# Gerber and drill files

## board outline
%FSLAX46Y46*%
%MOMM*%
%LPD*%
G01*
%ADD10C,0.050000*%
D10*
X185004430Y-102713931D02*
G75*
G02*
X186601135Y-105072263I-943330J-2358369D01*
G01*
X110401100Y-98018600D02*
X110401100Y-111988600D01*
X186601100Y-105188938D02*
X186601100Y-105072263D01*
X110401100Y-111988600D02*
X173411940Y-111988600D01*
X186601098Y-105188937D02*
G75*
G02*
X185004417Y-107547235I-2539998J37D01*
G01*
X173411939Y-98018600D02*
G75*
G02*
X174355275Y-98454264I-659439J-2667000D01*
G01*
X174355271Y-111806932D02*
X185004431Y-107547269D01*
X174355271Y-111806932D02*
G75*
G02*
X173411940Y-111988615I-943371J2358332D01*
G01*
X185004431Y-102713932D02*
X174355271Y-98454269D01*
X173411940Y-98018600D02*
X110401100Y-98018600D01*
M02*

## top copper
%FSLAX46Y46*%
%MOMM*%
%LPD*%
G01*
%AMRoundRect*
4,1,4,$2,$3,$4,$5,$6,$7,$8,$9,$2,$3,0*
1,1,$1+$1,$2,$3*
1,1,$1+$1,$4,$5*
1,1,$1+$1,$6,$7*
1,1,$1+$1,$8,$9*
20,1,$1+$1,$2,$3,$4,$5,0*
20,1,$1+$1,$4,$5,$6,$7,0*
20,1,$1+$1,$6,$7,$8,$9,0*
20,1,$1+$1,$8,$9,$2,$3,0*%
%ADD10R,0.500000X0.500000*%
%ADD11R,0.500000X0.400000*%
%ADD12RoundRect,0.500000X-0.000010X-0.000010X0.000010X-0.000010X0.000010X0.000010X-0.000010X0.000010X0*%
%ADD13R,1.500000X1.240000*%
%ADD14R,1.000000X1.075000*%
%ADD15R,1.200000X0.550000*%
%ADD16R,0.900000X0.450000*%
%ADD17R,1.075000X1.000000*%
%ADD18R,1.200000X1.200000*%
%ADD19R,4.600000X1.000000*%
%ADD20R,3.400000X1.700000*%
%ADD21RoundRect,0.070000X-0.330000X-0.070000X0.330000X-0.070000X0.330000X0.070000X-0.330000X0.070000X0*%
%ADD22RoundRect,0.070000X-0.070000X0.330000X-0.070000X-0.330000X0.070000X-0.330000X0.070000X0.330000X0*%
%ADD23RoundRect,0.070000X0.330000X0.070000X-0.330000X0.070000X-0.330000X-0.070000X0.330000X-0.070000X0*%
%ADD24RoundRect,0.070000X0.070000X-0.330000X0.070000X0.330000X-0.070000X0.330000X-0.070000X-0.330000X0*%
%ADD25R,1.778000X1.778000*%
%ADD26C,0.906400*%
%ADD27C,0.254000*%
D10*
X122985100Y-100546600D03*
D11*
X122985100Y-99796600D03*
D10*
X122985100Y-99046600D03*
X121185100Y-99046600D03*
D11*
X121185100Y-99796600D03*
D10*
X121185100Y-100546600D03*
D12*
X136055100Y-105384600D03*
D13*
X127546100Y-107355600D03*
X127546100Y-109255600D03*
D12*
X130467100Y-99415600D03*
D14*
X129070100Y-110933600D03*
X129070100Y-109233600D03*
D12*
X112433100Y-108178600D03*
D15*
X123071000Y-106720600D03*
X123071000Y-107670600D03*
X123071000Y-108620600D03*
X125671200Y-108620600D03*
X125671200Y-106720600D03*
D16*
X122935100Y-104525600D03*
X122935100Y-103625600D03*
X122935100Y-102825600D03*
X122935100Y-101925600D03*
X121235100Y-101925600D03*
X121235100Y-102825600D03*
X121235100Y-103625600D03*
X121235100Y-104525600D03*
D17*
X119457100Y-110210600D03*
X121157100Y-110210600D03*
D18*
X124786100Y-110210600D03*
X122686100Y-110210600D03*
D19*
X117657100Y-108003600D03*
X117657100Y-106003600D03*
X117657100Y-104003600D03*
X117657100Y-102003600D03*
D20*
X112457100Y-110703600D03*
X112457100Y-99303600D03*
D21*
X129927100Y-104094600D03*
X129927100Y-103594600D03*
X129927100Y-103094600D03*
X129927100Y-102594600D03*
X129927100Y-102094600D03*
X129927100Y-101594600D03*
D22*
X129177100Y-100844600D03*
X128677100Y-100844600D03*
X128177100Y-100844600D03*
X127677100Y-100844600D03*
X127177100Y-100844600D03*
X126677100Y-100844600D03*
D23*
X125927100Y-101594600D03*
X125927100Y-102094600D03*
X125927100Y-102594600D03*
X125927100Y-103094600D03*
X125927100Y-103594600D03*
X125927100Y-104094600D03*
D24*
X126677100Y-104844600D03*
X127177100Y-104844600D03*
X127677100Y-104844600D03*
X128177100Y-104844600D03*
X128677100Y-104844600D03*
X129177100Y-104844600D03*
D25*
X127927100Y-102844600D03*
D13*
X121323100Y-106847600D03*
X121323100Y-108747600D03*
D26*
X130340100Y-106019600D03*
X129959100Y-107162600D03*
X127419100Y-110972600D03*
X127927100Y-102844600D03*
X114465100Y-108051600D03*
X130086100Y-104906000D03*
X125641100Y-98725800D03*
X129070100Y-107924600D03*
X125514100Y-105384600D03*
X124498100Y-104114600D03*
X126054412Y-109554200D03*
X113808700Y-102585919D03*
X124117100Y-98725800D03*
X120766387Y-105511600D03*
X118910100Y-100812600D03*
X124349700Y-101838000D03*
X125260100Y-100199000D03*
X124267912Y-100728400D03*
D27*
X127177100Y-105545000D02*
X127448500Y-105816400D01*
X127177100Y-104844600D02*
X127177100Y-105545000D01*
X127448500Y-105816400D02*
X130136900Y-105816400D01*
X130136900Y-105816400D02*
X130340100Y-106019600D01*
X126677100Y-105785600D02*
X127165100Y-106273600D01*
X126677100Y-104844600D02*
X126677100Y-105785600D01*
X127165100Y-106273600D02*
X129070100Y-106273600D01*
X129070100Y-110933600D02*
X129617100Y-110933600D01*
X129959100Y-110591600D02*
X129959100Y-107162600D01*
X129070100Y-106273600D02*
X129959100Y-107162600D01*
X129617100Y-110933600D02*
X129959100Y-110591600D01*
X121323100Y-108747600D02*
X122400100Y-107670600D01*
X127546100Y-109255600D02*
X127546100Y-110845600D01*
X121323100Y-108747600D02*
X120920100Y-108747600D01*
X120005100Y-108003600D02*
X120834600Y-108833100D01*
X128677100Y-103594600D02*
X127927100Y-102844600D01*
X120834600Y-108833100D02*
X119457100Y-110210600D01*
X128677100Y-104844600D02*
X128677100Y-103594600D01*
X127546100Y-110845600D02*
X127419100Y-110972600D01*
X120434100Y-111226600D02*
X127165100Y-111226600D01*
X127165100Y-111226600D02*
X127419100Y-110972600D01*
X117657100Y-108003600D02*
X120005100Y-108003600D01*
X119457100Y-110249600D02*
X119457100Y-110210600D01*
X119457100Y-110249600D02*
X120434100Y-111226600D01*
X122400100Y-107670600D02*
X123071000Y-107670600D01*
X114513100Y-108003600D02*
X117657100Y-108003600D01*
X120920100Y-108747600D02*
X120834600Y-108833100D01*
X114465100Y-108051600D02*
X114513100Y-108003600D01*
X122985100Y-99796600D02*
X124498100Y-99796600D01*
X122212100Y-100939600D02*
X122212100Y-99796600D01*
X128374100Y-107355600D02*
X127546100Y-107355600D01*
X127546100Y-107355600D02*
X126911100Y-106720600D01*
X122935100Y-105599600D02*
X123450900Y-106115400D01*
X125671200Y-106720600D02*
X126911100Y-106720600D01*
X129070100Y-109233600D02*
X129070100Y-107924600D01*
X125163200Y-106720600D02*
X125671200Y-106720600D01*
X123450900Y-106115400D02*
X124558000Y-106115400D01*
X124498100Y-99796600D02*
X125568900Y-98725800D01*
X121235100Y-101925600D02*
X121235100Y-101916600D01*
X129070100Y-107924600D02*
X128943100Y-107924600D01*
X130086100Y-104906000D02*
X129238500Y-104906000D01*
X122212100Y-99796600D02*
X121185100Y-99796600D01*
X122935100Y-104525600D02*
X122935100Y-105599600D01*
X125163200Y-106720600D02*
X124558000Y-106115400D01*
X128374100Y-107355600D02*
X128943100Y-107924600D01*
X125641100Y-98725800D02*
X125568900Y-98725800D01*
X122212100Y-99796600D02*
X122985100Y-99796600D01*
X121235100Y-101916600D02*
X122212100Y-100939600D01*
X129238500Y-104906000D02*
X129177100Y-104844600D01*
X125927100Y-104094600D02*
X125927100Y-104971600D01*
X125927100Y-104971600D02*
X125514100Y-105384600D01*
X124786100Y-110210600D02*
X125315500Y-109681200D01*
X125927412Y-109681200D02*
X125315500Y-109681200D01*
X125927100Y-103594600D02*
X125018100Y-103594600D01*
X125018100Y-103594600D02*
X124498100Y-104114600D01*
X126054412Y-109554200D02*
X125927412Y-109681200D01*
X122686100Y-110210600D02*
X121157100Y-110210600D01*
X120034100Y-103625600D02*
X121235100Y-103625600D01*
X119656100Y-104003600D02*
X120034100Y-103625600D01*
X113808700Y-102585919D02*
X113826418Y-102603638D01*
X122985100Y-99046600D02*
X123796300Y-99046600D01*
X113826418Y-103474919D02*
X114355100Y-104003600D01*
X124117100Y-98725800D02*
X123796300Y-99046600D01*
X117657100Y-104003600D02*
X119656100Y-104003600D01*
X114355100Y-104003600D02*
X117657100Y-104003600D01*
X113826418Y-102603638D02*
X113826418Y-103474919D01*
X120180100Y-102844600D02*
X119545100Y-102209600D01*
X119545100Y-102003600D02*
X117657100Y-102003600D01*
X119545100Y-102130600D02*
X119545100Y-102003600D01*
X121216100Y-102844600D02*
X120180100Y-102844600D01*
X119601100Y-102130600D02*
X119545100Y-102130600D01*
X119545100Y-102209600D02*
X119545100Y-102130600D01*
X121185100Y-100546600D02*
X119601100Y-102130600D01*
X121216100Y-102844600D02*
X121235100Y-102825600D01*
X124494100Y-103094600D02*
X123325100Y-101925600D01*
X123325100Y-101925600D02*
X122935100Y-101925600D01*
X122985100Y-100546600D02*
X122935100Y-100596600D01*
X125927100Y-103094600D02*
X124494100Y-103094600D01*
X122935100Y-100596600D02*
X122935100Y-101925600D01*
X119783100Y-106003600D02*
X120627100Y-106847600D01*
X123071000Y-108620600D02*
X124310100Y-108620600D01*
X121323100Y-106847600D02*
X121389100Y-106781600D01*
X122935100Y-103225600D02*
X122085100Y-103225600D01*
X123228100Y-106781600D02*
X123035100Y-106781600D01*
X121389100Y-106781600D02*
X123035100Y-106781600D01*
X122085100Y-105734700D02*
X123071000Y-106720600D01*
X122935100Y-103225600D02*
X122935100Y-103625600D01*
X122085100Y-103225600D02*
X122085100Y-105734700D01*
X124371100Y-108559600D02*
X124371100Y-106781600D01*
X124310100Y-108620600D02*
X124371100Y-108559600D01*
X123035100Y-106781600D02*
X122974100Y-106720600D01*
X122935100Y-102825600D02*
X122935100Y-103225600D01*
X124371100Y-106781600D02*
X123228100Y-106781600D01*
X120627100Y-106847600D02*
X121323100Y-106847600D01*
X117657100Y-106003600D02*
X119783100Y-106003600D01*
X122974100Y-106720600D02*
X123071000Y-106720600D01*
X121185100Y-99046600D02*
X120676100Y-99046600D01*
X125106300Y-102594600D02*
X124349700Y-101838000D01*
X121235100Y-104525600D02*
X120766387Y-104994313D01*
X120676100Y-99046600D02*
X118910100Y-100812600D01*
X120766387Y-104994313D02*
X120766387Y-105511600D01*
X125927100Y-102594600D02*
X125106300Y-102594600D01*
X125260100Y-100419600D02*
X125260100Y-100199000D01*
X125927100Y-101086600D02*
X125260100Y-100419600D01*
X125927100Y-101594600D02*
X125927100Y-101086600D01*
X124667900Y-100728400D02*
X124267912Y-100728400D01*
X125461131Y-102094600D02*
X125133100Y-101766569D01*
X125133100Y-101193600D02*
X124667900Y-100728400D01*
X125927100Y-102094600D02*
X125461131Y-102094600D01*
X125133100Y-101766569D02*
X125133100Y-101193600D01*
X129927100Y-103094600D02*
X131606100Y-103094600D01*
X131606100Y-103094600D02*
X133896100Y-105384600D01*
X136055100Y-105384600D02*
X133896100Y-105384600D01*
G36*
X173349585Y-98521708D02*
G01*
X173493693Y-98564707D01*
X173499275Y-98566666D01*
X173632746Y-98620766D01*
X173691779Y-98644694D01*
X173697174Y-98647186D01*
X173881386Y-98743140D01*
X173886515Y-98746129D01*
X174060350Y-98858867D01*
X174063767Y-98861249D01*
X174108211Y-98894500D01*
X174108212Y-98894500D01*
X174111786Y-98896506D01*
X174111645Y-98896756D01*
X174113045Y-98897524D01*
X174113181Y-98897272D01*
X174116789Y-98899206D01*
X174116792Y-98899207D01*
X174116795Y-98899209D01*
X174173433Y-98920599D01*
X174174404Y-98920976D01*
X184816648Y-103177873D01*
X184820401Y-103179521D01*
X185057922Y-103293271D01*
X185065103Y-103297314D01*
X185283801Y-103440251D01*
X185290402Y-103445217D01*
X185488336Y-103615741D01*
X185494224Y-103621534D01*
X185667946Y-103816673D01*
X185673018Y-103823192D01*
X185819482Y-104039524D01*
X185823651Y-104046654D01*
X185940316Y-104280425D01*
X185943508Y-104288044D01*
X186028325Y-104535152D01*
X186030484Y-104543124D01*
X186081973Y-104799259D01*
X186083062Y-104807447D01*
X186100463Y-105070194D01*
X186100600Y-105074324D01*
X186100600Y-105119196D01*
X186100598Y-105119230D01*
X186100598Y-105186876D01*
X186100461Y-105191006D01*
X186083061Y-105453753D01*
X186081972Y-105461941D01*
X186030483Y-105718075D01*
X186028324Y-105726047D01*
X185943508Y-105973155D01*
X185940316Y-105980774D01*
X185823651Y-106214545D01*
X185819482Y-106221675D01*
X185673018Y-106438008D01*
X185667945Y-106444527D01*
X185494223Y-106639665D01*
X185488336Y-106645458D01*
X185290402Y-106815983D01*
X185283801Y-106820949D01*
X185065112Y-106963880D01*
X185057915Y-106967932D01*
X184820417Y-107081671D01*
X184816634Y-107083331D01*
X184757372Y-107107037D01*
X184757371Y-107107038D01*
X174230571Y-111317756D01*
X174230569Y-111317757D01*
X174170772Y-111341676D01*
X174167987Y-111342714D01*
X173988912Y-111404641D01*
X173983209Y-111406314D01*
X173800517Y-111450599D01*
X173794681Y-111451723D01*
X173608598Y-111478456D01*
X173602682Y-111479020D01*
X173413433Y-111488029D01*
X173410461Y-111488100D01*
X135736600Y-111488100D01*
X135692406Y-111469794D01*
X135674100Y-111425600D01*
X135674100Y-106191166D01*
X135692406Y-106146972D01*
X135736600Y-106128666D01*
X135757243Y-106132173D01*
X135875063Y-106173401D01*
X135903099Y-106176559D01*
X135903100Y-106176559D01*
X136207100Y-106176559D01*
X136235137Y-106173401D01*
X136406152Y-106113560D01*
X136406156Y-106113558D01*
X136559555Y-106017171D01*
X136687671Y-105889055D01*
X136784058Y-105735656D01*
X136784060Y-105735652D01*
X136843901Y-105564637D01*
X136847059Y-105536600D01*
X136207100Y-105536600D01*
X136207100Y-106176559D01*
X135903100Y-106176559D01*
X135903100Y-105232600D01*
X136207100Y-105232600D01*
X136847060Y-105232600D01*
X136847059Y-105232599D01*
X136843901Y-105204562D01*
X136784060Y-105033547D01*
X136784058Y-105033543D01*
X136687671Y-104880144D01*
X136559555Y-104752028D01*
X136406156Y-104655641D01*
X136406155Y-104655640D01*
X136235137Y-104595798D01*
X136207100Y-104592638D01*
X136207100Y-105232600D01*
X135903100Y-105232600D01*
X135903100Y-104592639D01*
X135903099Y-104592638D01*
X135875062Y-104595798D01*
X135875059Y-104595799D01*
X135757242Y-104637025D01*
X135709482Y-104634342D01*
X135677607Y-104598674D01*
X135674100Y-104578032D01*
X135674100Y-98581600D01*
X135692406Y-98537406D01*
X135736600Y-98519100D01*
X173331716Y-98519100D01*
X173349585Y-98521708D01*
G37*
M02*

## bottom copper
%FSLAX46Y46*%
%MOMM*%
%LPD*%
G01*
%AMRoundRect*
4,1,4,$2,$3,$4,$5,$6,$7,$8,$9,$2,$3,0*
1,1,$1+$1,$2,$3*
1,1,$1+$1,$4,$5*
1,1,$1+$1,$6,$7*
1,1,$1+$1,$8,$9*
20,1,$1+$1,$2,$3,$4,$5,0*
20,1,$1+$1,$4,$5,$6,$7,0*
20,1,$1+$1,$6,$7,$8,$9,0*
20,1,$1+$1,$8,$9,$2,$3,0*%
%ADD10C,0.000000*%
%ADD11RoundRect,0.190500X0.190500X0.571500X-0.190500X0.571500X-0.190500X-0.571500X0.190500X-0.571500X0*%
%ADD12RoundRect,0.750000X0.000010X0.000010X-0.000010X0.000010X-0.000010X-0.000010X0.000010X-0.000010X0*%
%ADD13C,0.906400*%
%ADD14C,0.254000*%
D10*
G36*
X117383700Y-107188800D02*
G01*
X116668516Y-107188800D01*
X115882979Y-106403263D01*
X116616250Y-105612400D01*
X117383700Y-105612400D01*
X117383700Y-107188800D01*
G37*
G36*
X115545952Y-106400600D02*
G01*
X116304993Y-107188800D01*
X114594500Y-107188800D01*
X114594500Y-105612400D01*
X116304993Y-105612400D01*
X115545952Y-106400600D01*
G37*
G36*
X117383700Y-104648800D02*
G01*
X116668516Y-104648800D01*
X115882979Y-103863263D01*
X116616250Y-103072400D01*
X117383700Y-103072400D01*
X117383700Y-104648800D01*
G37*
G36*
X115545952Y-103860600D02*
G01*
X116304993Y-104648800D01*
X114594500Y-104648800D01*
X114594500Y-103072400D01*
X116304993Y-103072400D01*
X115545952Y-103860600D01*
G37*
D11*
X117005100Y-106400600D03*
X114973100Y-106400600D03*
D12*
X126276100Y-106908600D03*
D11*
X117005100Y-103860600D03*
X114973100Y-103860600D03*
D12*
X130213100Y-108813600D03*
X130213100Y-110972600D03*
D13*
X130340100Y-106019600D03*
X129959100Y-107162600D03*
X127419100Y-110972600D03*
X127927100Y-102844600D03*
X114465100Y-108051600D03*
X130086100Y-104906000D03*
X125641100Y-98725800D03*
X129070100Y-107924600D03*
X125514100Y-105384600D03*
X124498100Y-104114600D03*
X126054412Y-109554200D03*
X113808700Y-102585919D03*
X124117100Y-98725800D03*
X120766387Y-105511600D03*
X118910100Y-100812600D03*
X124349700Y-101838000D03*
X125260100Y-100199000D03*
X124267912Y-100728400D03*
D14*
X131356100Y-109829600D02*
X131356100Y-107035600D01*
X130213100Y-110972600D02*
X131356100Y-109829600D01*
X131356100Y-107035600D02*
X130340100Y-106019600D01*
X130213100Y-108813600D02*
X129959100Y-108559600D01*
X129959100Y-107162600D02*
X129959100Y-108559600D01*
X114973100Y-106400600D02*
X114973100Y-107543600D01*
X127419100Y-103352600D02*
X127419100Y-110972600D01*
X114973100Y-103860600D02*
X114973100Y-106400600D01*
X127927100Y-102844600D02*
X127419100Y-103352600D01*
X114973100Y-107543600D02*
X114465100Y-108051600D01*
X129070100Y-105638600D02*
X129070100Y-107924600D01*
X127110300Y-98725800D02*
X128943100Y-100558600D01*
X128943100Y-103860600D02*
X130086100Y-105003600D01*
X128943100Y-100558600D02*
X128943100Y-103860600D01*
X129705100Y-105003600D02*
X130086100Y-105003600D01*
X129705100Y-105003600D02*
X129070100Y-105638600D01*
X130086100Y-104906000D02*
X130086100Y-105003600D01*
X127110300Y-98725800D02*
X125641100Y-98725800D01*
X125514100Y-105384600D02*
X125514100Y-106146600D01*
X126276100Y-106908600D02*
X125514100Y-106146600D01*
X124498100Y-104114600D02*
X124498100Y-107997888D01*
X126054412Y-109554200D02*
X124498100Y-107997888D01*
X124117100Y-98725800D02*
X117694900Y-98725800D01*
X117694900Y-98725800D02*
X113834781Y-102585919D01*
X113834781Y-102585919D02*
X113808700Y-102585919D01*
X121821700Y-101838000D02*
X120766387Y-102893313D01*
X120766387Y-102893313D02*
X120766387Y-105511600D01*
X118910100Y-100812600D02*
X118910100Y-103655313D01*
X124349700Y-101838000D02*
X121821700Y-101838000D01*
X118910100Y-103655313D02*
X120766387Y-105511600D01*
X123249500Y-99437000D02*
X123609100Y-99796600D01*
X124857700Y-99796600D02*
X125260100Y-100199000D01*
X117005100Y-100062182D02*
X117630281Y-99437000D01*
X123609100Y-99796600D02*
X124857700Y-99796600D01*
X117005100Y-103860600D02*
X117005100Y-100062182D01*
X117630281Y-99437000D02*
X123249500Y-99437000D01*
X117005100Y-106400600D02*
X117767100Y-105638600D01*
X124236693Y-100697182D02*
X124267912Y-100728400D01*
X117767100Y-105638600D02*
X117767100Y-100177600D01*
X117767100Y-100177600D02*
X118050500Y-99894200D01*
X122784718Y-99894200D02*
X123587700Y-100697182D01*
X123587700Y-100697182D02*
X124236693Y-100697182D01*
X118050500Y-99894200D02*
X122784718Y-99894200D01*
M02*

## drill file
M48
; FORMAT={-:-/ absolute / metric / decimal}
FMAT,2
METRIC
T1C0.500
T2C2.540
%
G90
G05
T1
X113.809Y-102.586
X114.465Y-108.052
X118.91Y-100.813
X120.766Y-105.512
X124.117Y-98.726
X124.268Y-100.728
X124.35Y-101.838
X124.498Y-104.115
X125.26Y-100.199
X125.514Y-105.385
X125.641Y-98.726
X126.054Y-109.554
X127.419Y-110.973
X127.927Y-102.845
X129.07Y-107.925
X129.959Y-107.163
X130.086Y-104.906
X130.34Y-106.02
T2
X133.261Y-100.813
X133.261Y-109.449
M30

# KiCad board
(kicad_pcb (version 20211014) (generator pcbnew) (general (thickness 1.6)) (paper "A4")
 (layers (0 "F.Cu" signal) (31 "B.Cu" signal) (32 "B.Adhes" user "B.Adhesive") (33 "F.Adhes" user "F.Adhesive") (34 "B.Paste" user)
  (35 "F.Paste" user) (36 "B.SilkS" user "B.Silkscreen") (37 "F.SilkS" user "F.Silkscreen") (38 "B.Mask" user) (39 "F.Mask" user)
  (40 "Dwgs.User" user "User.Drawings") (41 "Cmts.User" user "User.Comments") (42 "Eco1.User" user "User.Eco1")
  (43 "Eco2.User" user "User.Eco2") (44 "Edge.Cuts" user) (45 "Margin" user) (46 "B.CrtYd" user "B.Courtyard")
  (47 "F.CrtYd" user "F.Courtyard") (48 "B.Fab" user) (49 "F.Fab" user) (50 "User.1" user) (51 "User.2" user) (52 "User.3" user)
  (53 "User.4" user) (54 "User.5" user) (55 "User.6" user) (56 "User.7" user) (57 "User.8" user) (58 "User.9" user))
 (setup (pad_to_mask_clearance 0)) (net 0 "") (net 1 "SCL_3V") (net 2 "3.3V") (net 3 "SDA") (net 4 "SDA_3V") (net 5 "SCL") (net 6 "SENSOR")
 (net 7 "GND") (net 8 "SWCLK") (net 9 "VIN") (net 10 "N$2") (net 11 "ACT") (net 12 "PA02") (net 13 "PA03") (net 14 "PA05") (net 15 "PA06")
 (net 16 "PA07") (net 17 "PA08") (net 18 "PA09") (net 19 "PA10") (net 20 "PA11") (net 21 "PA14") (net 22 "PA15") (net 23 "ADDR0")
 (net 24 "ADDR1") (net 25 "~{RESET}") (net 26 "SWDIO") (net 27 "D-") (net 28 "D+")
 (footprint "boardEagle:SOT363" (layer "F.Cu") (at 122.0851 99.7966 90)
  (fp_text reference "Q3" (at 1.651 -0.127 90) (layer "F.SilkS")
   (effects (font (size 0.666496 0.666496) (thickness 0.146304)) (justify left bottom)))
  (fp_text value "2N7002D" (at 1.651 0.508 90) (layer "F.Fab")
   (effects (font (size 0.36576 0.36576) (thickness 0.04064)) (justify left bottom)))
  (pad "1" smd rect (at -0.75 0.9 90) (size 0.5 0.5) (layers "F.Cu" "F.Paste" "F.Mask") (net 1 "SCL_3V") (solder_mask_margin 0.0508))
  (pad "2" smd rect (at 0 0.9 90) (size 0.4 0.5) (layers "F.Cu" "F.Paste" "F.Mask") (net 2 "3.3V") (solder_mask_margin 0.0508))
  (pad "3" smd rect (at 0.75 0.9 90) (size 0.5 0.5) (layers "F.Cu" "F.Paste" "F.Mask") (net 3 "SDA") (solder_mask_margin 0.0508))
  (pad "4" smd rect (at 0.75 -0.9 90) (size 0.5 0.5) (layers "F.Cu" "F.Paste" "F.Mask") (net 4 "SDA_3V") (solder_mask_margin 0.0508))
  (pad "5" smd rect (at 0 -0.9 90) (size 0.4 0.5) (layers "F.Cu" "F.Paste" "F.Mask") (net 2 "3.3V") (solder_mask_margin 0.0508))
  (pad "6" smd rect (at -0.75 -0.9 90) (size 0.5 0.5) (layers "F.Cu" "F.Paste" "F.Mask") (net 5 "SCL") (solder_mask_margin 0.0508)))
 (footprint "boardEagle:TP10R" (layer "F.Cu") (at 136.0551 105.3846)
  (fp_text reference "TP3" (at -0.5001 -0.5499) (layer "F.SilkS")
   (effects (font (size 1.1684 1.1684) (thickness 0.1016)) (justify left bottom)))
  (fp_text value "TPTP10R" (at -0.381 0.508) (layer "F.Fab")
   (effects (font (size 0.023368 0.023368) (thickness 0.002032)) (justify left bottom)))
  (pad "TP" smd roundrect (at 0 0) (size 1 1) (layers "F.Cu" "F.Mask") (roundrect_rratio 0.5) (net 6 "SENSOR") (solder_mask_margin 0.0508)))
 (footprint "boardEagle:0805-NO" (layer "F.Cu") (at 127.5461 108.3056 -90)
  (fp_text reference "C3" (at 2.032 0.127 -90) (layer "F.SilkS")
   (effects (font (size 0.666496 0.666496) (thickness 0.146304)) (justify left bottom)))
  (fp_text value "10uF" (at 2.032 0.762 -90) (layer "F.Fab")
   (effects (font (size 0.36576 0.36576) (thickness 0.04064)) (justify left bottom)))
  (pad "1" smd rect (at -0.95 0 270) (size 1.24 1.5) (layers "F.Cu" "F.Paste" "F.Mask") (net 2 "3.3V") (solder_mask_margin 0.0508))
  (pad "2" smd rect (at 0.95 0 270) (size 1.24 1.5) (layers "F.Cu" "F.Paste" "F.Mask") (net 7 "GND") (solder_mask_margin 0.0508)))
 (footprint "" (layer "F.Cu") (at 133.2611 100.8126)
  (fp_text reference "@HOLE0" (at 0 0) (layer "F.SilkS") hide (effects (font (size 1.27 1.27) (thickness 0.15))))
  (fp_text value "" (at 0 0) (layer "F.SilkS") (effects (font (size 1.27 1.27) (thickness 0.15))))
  (pad "" np_thru_hole circle (at 0 0) (size 2.54 2.54) (drill 2.54) (layers *.Cu *.Mask)))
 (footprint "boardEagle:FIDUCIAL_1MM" (layer "F.Cu") (at 130.4671 99.4156)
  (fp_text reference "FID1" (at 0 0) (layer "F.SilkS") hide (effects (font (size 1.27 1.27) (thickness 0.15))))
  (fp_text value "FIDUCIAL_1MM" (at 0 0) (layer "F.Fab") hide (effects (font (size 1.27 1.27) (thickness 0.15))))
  (pad "1" smd roundrect (at 0 0) (size 1 1) (layers "F.Cu" "F.Mask") (roundrect_rratio 0.5) (solder_mask_margin 0.0508)))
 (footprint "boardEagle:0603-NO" (layer "F.Cu") (at 129.0701 110.0836 90)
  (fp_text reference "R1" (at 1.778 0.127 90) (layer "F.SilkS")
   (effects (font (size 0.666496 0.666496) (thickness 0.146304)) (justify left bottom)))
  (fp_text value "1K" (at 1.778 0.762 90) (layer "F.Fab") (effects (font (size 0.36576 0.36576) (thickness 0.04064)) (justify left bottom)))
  (pad "1" smd rect (at -0.85 0 90) (size 1.075 1) (layers "F.Cu" "F.Paste" "F.Mask") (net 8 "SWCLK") (solder_mask_margin 0.0508))
  (pad "2" smd rect (at 0.85 0 90) (size 1.075 1) (layers "F.Cu" "F.Paste" "F.Mask") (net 2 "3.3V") (solder_mask_margin 0.0508)))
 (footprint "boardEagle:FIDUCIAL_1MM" (layer "F.Cu") (at 112.4331 108.1786)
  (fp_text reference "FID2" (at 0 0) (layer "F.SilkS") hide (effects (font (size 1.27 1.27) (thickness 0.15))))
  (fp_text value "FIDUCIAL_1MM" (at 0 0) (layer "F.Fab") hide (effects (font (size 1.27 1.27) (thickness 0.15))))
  (pad "1" smd roundrect (at 0 0) (size 1 1) (layers "F.Cu" "F.Mask") (roundrect_rratio 0.5) (solder_mask_margin 0.0508)))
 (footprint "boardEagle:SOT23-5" (layer "F.Cu") (at 124.3711 107.6706 -90)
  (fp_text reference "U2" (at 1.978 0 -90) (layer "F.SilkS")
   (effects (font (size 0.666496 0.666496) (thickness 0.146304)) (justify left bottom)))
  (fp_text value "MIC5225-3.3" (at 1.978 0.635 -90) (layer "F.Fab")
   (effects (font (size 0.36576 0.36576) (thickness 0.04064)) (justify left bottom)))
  (pad "1" smd rect (at -0.95 1.3001 270) (size 0.55 1.2) (layers "F.Cu" "F.Paste" "F.Mask") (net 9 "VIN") (solder_mask_margin 0.0508))
  (pad "2" smd rect (at 0 1.3001 270) (size 0.55 1.2) (layers "F.Cu" "F.Paste" "F.Mask") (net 7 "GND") (solder_mask_margin 0.0508))
  (pad "3" smd rect (at 0.95 1.3001 270) (size 0.55 1.2) (layers "F.Cu" "F.Paste" "F.Mask") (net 9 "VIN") (solder_mask_margin 0.0508))
  (pad "4" smd rect (at 0.95 -1.3001 270) (size 0.55 1.2) (layers "F.Cu" "F.Paste" "F.Mask") (solder_mask_margin 0.0508))
  (pad "5" smd rect (at -0.95 -1.3001 270) (size 0.55 1.2) (layers "F.Cu" "F.Paste" "F.Mask") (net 2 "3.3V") (solder_mask_margin 0.0508)))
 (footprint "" (layer "F.Cu") (at 133.2611 109.4486)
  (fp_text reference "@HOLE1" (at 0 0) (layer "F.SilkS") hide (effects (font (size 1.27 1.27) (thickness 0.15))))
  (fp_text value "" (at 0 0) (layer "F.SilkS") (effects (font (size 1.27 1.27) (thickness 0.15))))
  (pad "" np_thru_hole circle (at 0 0) (size 2.54 2.54) (drill 2.54) (layers *.Cu *.Mask)))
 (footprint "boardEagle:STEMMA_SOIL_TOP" (layer "F.Cu") (at 110.4011 111.9886)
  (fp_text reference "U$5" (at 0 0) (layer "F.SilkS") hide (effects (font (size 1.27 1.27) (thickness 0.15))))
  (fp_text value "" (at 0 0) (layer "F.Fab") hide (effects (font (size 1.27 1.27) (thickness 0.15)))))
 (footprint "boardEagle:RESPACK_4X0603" (layer "F.Cu") (at 122.0851 103.2256 90)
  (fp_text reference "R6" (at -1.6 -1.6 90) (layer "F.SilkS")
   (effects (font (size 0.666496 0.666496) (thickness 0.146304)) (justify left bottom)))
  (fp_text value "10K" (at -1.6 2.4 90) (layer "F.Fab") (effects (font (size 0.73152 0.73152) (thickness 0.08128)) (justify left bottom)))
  (pad "1" smd rect (at -1.3 0.85 90) (size 0.45 0.9) (layers "F.Cu" "F.Paste" "F.Mask") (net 2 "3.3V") (solder_mask_margin 0.0508))
  (pad "2" smd rect (at -0.4 0.85 90) (size 0.45 0.9) (layers "F.Cu" "F.Paste" "F.Mask") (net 9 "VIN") (solder_mask_margin 0.0508))
  (pad "3" smd rect (at 0.4 0.85 90) (size 0.45 0.9) (layers "F.Cu" "F.Paste" "F.Mask") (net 9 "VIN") (solder_mask_margin 0.0508))
  (pad "4" smd rect (at 1.3 0.85 90) (size 0.45 0.9) (layers "F.Cu" "F.Paste" "F.Mask") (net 1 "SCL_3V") (solder_mask_margin 0.0508))
  (pad "5" smd rect (at 1.3 -0.85 90) (size 0.45 0.9) (layers "F.Cu" "F.Paste" "F.Mask") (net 2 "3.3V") (solder_mask_margin 0.0508))
  (pad "6" smd rect (at 0.4 -0.85 90) (size 0.45 0.9) (layers "F.Cu" "F.Paste" "F.Mask") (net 5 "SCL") (solder_mask_margin 0.0508))
  (pad "7" smd rect (at -0.4 -0.85 90) (size 0.45 0.9) (layers "F.Cu" "F.Paste" "F.Mask") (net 3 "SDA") (solder_mask_margin 0.0508))
  (pad "8" smd rect (at -1.3 -0.85 90) (size 0.45 0.9) (layers "F.Cu" "F.Paste" "F.Mask") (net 4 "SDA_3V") (solder_mask_margin 0.0508)))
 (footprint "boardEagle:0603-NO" (layer "F.Cu") (at 120.3071 110.2106)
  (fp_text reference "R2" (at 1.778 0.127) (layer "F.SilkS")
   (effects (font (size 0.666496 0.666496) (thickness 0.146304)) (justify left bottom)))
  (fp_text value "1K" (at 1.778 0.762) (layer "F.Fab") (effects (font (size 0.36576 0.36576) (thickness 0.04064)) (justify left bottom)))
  (pad "1" smd rect (at -0.85 0) (size 1.075 1) (layers "F.Cu" "F.Paste" "F.Mask") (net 7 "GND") (solder_mask_margin 0.0508))
  (pad "2" smd rect (at 0.85 0) (size 1.075 1) (layers "F.Cu" "F.Paste" "F.Mask") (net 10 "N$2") (solder_mask_margin 0.0508)))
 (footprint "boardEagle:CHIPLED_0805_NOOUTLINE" (layer "F.Cu") (at 123.7361 110.2106 90)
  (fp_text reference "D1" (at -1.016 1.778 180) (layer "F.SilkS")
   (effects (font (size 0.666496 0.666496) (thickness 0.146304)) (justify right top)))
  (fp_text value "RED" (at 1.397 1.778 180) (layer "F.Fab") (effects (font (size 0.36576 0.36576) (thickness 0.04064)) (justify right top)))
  (pad "A" smd rect (at 0 1.05 90) (size 1.2 1.2) (layers "F.Cu" "F.Paste" "F.Mask") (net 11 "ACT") (solder_mask_margin 0.0508))
  (pad "C" smd rect (at 0 -1.05 90) (size 1.2 1.2) (layers "F.Cu" "F.Paste" "F.Mask") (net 10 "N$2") (solder_mask_margin 0.0508)))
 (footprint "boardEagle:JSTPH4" (layer "F.Cu") (at 113.9571 105.0036 90)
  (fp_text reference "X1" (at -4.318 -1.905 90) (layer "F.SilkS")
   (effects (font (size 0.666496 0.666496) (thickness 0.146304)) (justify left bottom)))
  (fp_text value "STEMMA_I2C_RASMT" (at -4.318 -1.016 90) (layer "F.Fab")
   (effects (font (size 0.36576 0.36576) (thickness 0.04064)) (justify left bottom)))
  (pad "1" smd rect (at -3 3.7 90) (size 1 4.6) (layers "F.Cu" "F.Paste" "F.Mask") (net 7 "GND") (solder_mask_margin 0.0508))
  (pad "2" smd rect (at -1 3.7 90) (size 1 4.6) (layers "F.Cu" "F.Paste" "F.Mask") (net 9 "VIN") (solder_mask_margin 0.0508))
  (pad "3" smd rect (at 1 3.7 90) (size 1 4.6) (layers "F.Cu" "F.Paste" "F.Mask") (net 3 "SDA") (solder_mask_margin 0.0508))
  (pad "4" smd rect (at 3 3.7 90) (size 1 4.6) (layers "F.Cu" "F.Paste" "F.Mask") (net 5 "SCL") (solder_mask_margin 0.0508))
  (pad "NC1" smd rect (at -5.7 -1.5 180) (size 3.4 1.7) (layers "F.Cu" "F.Paste" "F.Mask") (solder_mask_margin 0.0508))
  (pad "NC2" smd rect (at 5.7 -1.5 180) (size 3.4 1.7) (layers "F.Cu" "F.Paste" "F.Mask") (solder_mask_margin 0.0508)))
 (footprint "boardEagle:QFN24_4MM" (layer "F.Cu") (at 127.9271 102.8446 180)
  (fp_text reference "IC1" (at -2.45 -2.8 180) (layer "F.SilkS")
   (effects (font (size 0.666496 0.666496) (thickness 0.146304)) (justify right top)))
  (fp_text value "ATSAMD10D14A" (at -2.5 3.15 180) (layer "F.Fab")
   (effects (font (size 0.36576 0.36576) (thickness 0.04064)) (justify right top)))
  (pad "1" smd roundrect (at -2 -1.25) (size 0.8 0.28) (layers "F.Cu" "F.Paste" "F.Mask") (roundrect_rratio 0.25) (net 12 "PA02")
   (solder_mask_margin 0.0508))
  (pad "2" smd roundrect (at -2 -0.75) (size 0.8 0.28) (layers "F.Cu" "F.Paste" "F.Mask") (roundrect_rratio 0.25) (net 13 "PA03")
   (solder_mask_margin 0.0508))
  (pad "3" smd roundrect (at -2 -0.25) (size 0.8 0.28) (layers "F.Cu" "F.Paste" "F.Mask") (roundrect_rratio 0.25) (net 6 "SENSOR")
   (solder_mask_margin 0.0508))
  (pad "4" smd roundrect (at -2 0.25) (size 0.8 0.28) (layers "F.Cu" "F.Paste" "F.Mask") (roundrect_rratio 0.25) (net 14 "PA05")
   (solder_mask_margin 0.0508))
  (pad "5" smd roundrect (at -2 0.75) (size 0.8 0.28) (layers "F.Cu" "F.Paste" "F.Mask") (roundrect_rratio 0.25) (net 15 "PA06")
   (solder_mask_margin 0.0508))
  (pad "6" smd roundrect (at -2 1.25) (size 0.8 0.28) (layers "F.Cu" "F.Paste" "F.Mask") (roundrect_rratio 0.25) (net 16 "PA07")
   (solder_mask_margin 0.0508))
  (pad "7" smd roundrect (at -1.25 2 270) (size 0.8 0.28) (layers "F.Cu" "F.Paste" "F.Mask") (roundrect_rratio 0.25) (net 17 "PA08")
   (solder_mask_margin 0.0508))
  (pad "8" smd roundrect (at -0.75 2 270) (size 0.8 0.28) (layers "F.Cu" "F.Paste" "F.Mask") (roundrect_rratio 0.25) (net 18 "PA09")
   (solder_mask_margin 0.0508))
  (pad "9" smd roundrect (at -0.25 2 270) (size 0.8 0.28) (layers "F.Cu" "F.Paste" "F.Mask") (roundrect_rratio 0.25) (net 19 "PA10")
   (solder_mask_margin 0.0508))
  (pad "10" smd roundrect (at 0.25 2 270) (size 0.8 0.28) (layers "F.Cu" "F.Paste" "F.Mask") (roundrect_rratio 0.25) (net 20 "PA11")
   (solder_mask_margin 0.0508))
  (pad "11" smd roundrect (at 0.75 2 270) (size 0.8 0.28) (layers "F.Cu" "F.Paste" "F.Mask") (roundrect_rratio 0.25) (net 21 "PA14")
   (solder_mask_margin 0.0508))
  (pad "12" smd roundrect (at 1.25 2 270) (size 0.8 0.28) (layers "F.Cu" "F.Paste" "F.Mask") (roundrect_rratio 0.25) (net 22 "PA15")
   (solder_mask_margin 0.0508))
  (pad "13" smd roundrect (at 2 1.25 180) (size 0.8 0.28) (layers "F.Cu" "F.Paste" "F.Mask") (roundrect_rratio 0.25) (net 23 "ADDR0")
   (solder_mask_margin 0.0508))
  (pad "14" smd roundrect (at 2 0.75 180) (size 0.8 0.28) (layers "F.Cu" "F.Paste" "F.Mask") (roundrect_rratio 0.25) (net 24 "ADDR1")
   (solder_mask_margin 0.0508))
  (pad "15" smd roundrect (at 2 0.25 180) (size 0.8 0.28) (layers "F.Cu" "F.Paste" "F.Mask") (roundrect_rratio 0.25) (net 4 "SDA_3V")
   (solder_mask_margin 0.0508))
  (pad "16" smd roundrect (at 2 -0.25 180) (size 0.8 0.28) (layers "F.Cu" "F.Paste" "F.Mask") (roundrect_rratio 0.25) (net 1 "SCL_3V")
   (solder_mask_margin 0.0508))
  (pad "17" smd roundrect (at 2 -0.75 180) (size 0.8 0.28) (layers "F.Cu" "F.Paste" "F.Mask") (roundrect_rratio 0.25) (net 11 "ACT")
   (solder_mask_margin 0.0508))
  (pad "18" smd roundrect (at 2 -1.25 180) (size 0.8 0.28) (layers "F.Cu" "F.Paste" "F.Mask") (roundrect_rratio 0.25) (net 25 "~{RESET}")
   (solder_mask_margin 0.0508))
  (pad "19" smd roundrect (at 1.25 -2 90) (size 0.8 0.28) (layers "F.Cu" "F.Paste" "F.Mask") (roundrect_rratio 0.25) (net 8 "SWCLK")
   (solder_mask_margin 0.0508))
  (pad "20" smd roundrect (at 0.75 -2 90) (size 0.8 0.28) (layers "F.Cu" "F.Paste" "F.Mask") (roundrect_rratio 0.25) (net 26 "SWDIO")
   (solder_mask_margin 0.0508))
  (pad "21" smd roundrect (at 0.25 -2 90) (size 0.8 0.28) (layers "F.Cu" "F.Paste" "F.Mask") (roundrect_rratio 0.25) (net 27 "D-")
   (solder_mask_margin 0.0508))
  (pad "22" smd roundrect (at -0.25 -2 90) (size 0.8 0.28) (layers "F.Cu" "F.Paste" "F.Mask") (roundrect_rratio 0.25) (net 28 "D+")
   (solder_mask_margin 0.0508))
  (pad "23" smd roundrect (at -0.75 -2 90) (size 0.8 0.28) (layers "F.Cu" "F.Paste" "F.Mask") (roundrect_rratio 0.25) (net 7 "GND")
   (solder_mask_margin 0.0508))
  (pad "24" smd roundrect (at -1.25 -2 90) (size 0.8 0.28) (layers "F.Cu" "F.Paste" "F.Mask") (roundrect_rratio 0.25) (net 2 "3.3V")
   (solder_mask_margin 0.0508))
  (pad "THERM" smd rect (at 0 0 180) (size 1.778 1.778) (layers "F.Cu" "F.Mask") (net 7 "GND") (solder_mask_margin 0.0508)))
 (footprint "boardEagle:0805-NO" (layer "F.Cu") (at 121.3231 107.7976 -90)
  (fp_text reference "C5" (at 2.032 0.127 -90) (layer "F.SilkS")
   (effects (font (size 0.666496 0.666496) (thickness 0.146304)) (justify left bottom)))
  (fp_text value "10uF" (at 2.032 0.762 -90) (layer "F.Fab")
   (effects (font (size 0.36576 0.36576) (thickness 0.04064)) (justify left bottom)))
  (pad "1" smd rect (at -0.95 0 270) (size 1.24 1.5) (layers "F.Cu" "F.Paste" "F.Mask") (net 9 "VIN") (solder_mask_margin 0.0508))
  (pad "2" smd rect (at 0.95 0 270) (size 1.24 1.5) (layers "F.Cu" "F.Paste" "F.Mask") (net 7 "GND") (solder_mask_margin 0.0508)))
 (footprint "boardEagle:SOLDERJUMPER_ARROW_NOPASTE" (layer "B.Cu") (at 115.9891 106.4006 180)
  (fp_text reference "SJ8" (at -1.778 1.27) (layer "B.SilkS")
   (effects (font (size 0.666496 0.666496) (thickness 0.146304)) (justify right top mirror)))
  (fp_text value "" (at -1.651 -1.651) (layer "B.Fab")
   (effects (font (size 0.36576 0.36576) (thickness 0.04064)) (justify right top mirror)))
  (fp_poly
   (pts (xy 0.106121 -0.002663) (xy -0.679416 -0.7882) (xy -1.3946 -0.7882) (xy -1.3946 0.7882) (xy -0.62715 0.7882)) (layer "B.Cu")
   (width 0) (fill solid))
  (fp_poly
   (pts (xy 1.3946 -0.7882) (xy -0.315893 -0.7882) (xy 0.443148 0) (xy -0.315893 0.7882) (xy 1.3946 0.7882)) (layer "B.Cu") (width 0)
   (fill solid))
  (pad "1" smd roundrect (at -1.016 0 180) (size 0.762 1.524) (layers "B.Cu") (roundrect_rratio 0.25) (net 24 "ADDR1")
   (solder_mask_margin 0.0508))
  (pad "2" smd roundrect (at 1.016 0 180) (size 0.762 1.524) (layers "B.Cu") (roundrect_rratio 0.25) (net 7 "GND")
   (solder_mask_margin 0.0508)))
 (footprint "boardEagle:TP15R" (layer "B.Cu") (at 126.2761 106.9086 180)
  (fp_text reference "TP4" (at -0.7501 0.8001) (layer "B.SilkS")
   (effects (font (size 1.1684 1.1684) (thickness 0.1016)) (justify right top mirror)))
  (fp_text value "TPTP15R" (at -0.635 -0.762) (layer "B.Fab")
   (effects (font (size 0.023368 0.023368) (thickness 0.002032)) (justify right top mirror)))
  (pad "TP" smd roundrect (at 0 0 180) (size 1.5 1.5) (layers "B.Cu" "B.Mask") (roundrect_rratio 0.5) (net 25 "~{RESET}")
   (solder_mask_margin 0.0508)))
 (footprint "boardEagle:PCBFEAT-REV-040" (layer "B.Cu") (at 119.0371 106.5276 180)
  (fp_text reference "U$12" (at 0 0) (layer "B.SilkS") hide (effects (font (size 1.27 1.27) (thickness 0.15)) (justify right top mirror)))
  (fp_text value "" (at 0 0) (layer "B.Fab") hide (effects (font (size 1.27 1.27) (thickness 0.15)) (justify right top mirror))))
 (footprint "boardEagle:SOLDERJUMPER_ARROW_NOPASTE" (layer "B.Cu") (at 115.9891 103.8606 180)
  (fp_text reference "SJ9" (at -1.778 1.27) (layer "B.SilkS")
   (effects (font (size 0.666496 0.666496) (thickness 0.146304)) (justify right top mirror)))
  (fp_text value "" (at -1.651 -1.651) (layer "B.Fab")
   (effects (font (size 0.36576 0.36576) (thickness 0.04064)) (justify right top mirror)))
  (fp_poly
   (pts (xy 0.106121 -0.002663) (xy -0.679416 -0.7882) (xy -1.3946 -0.7882) (xy -1.3946 0.7882) (xy -0.62715 0.7882)) (layer "B.Cu")
   (width 0) (fill solid))
  (fp_poly
   (pts (xy 1.3946 -0.7882) (xy -0.315893 -0.7882) (xy 0.443148 0) (xy -0.315893 0.7882) (xy 1.3946 0.7882)) (layer "B.Cu") (width 0)
   (fill solid))
  (pad "1" smd roundrect (at -1.016 0 180) (size 0.762 1.524) (layers "B.Cu") (roundrect_rratio 0.25) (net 23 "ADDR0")
   (solder_mask_margin 0.0508))
  (pad "2" smd roundrect (at 1.016 0 180) (size 0.762 1.524) (layers "B.Cu") (roundrect_rratio 0.25) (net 7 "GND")
   (solder_mask_margin 0.0508)))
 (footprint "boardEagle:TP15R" (layer "B.Cu") (at 130.2131 108.8136 180)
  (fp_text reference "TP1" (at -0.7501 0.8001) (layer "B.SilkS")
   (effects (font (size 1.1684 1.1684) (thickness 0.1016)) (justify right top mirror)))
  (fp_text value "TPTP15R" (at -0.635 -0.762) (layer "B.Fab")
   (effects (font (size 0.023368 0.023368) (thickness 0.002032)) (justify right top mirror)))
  (pad "TP" smd roundrect (at 0 0 180) (size 1.5 1.5) (layers "B.Cu" "B.Mask") (roundrect_rratio 0.5) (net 8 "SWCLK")
   (solder_mask_margin 0.0508)))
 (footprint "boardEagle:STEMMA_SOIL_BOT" (layer "B.Cu") (at 186.7281 111.9886 180)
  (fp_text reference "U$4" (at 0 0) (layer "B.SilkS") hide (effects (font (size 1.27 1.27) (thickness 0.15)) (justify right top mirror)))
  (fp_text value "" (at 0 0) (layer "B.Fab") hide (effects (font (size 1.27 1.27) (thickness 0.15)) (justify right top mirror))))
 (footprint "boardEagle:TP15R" (layer "B.Cu") (at 130.2131 110.9726 180)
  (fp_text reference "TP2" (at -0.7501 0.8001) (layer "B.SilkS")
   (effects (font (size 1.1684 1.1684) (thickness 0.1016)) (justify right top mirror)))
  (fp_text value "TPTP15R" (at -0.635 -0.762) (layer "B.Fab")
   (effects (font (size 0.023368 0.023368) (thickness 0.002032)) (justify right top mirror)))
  (pad "TP" smd roundrect (at 0 0 180) (size 1.5 1.5) (layers "B.Cu" "B.Mask") (roundrect_rratio 0.5) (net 26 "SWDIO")
   (solder_mask_margin 0.0508)))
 (gr_arc (start 185.00443 102.713931) (mid 186.16439 103.648265) (end 186.6011 105.072263) (layer "Edge.Cuts") (width 0.05))
 (gr_line (start 110.4011 98.0186) (end 110.4011 111.9886) (layer "Edge.Cuts") (width 0.05))
 (gr_line (start 186.6011 105.188938) (end 186.6011 105.072263) (layer "Edge.Cuts") (width 0.05))
 (gr_line (start 110.4011 111.9886) (end 173.41194 111.9886) (layer "Edge.Cuts") (width 0.05))
 (gr_arc (start 186.601098 105.188937) (mid 186.16439 106.612935) (end 185.004431 107.547269) (layer "Edge.Cuts") (width 0.05))
 (gr_arc (start 173.411939 98.0186) (mid 173.90439 98.191431) (end 174.355271 98.454269) (layer "Edge.Cuts") (width 0.05))
 (gr_line (start 174.355271 111.806932) (end 185.004431 107.547269) (layer "Edge.Cuts") (width 0.05))
 (gr_arc (start 174.355271 111.806932) (mid 173.892272 111.94277) (end 173.41194 111.9886) (layer "Edge.Cuts") (width 0.05))
 (gr_line (start 185.004431 102.713932) (end 174.355271 98.454269) (layer "Edge.Cuts") (width 0.05))
 (gr_line (start 173.41194 98.0186) (end 110.4011 98.0186) (layer "Edge.Cuts") (width 0.05))
 (segment (start 127.1771 105.545) (end 127.4485 105.8164) (width 0.254) (layer "F.Cu") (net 26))
 (segment (start 127.1771 104.8446) (end 127.1771 105.545) (width 0.254) (layer "F.Cu") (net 26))
 (segment (start 127.4485 105.8164) (end 130.1369 105.8164) (width 0.254) (layer "F.Cu") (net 26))
 (segment (start 130.1369 105.8164) (end 130.3401 106.0196) (width 0.254) (layer "F.Cu") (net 26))
 (via (at 130.3401 106.0196) (size 0.9064) (drill 0.5) (layers "F.Cu" "B.Cu") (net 26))
 (segment (start 131.3561 109.8296) (end 131.3561 107.0356) (width 0.254) (layer "B.Cu") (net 26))
 (segment (start 130.2131 110.9726) (end 131.3561 109.8296) (width 0.254) (layer "B.Cu") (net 26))
 (segment (start 131.3561 107.0356) (end 130.3401 106.0196) (width 0.254) (layer "B.Cu") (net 26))
 (segment (start 126.6771 105.7856) (end 127.1651 106.2736) (width 0.254) (layer "F.Cu") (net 8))
 (segment (start 126.6771 104.8446) (end 126.6771 105.7856) (width 0.254) (layer "F.Cu") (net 8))
 (segment (start 127.1651 106.2736) (end 129.0701 106.2736) (width 0.254) (layer "F.Cu") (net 8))
 (segment (start 129.0701 110.9336) (end 129.6171 110.9336) (width 0.254) (layer "F.Cu") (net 8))
 (segment (start 129.9591 110.5916) (end 129.9591 107.1626) (width 0.254) (layer "F.Cu") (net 8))
 (segment (start 129.0701 106.2736) (end 129.9591 107.1626) (width 0.254) (layer "F.Cu") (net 8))
 (segment (start 129.6171 110.9336) (end 129.9591 110.5916) (width 0.254) (layer "F.Cu") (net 8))
 (via (at 129.9591 107.1626) (size 0.9064) (drill 0.5) (layers "F.Cu" "B.Cu") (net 8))
 (segment (start 130.2131 108.8136) (end 129.9591 108.5596) (width 0.254) (layer "B.Cu") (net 8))
 (segment (start 129.9591 107.1626) (end 129.9591 108.5596) (width 0.254) (layer "B.Cu") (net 8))
 (segment (start 121.3231 108.7476) (end 122.4001 107.6706) (width 0.254) (layer "F.Cu") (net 7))
 (segment (start 127.5461 109.2556) (end 127.5461 110.8456) (width 0.254) (layer "F.Cu") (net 7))
 (segment (start 121.3231 108.7476) (end 120.9201 108.7476) (width 0.254) (layer "F.Cu") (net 7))
 (segment (start 120.0051 108.0036) (end 120.8346 108.8331) (width 0.254) (layer "F.Cu") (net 7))
 (segment (start 128.6771 103.5946) (end 127.9271 102.8446) (width 0.254) (layer "F.Cu") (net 7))
 (segment (start 120.8346 108.8331) (end 119.4571 110.2106) (width 0.254) (layer "F.Cu") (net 7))
 (segment (start 128.6771 104.8446) (end 128.6771 103.5946) (width 0.254) (layer "F.Cu") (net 7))
 (segment (start 127.5461 110.8456) (end 127.4191 110.9726) (width 0.254) (layer "F.Cu") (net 7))
 (segment (start 120.4341 111.2266) (end 127.1651 111.2266) (width 0.254) (layer "F.Cu") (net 7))
 (segment (start 127.1651 111.2266) (end 127.4191 110.9726) (width 0.254) (layer "F.Cu") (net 7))
 (segment (start 117.6571 108.0036) (end 120.0051 108.0036) (width 0.254) (layer "F.Cu") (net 7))
 (segment (start 119.4571 110.2496) (end 119.4571 110.2106) (width 0.254) (layer "F.Cu") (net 7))
 (segment (start 119.4571 110.2496) (end 120.4341 111.2266) (width 0.254) (layer "F.Cu") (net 7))
 (segment (start 122.4001 107.6706) (end 123.071 107.6706) (width 0.254) (layer "F.Cu") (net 7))
 (segment (start 114.5131 108.0036) (end 117.6571 108.0036) (width 0.254) (layer "F.Cu") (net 7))
 (segment (start 120.9201 108.7476) (end 120.8346 108.8331) (width 0.254) (layer "F.Cu") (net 7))
 (segment (start 114.4651 108.0516) (end 114.5131 108.0036) (width 0.254) (layer "F.Cu") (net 7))
 (via (at 127.4191 110.9726) (size 0.9064) (drill 0.5) (layers "F.Cu" "B.Cu") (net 7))
 (via (at 127.9271 102.8446) (size 0.9064) (drill 0.5) (layers "F.Cu" "B.Cu") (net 7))
 (via (at 114.4651 108.0516) (size 0.9064) (drill 0.5) (layers "F.Cu" "B.Cu") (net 7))
 (segment (start 114.9731 106.4006) (end 114.9731 107.5436) (width 0.254) (layer "B.Cu") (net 7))
 (segment (start 127.4191 103.3526) (end 127.4191 110.9726) (width 0.254) (layer "B.Cu") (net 7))
 (segment (start 114.9731 103.8606) (end 114.9731 106.4006) (width 0.254) (layer "B.Cu") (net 7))
 (segment (start 127.9271 102.8446) (end 127.4191 103.3526) (width 0.254) (layer "B.Cu") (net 7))
 (segment (start 114.9731 107.5436) (end 114.4651 108.0516) (width 0.254) (layer "B.Cu") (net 7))
 (segment (start 122.9851 99.7966) (end 124.4981 99.7966) (width 0.254) (layer "F.Cu") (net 2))
 (segment (start 122.2121 100.9396) (end 122.2121 99.7966) (width 0.254) (layer "F.Cu") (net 2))
 (segment (start 128.3741 107.3556) (end 127.5461 107.3556) (width 0.254) (layer "F.Cu") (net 2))
 (segment (start 127.5461 107.3556) (end 126.9111 106.7206) (width 0.254) (layer "F.Cu") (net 2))
 (segment (start 122.9351 105.5996) (end 123.4509 106.1154) (width 0.254) (layer "F.Cu") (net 2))
 (segment (start 125.6712 106.7206) (end 126.9111 106.7206) (width 0.254) (layer "F.Cu") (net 2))
 (segment (start 129.0701 109.2336) (end 129.0701 107.9246) (width 0.254) (layer "F.Cu") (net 2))
 (segment (start 125.1632 106.7206) (end 125.6712 106.7206) (width 0.254) (layer "F.Cu") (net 2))
 (segment (start 123.4509 106.1154) (end 124.558 106.1154) (width 0.254) (layer "F.Cu") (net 2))
 (segment (start 124.4981 99.7966) (end 125.5689 98.7258) (width 0.254) (layer "F.Cu") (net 2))
 (segment (start 121.2351 101.9256) (end 121.2351 101.9166) (width 0.254) (layer "F.Cu") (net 2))
 (segment (start 129.0701 107.9246) (end 128.9431 107.9246) (width 0.254) (layer "F.Cu") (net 2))
 (segment (start 130.0861 104.906) (end 129.2385 104.906) (width 0.254) (layer "F.Cu") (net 2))
 (segment (start 122.2121 99.7966) (end 121.1851 99.7966) (width 0.254) (layer "F.Cu") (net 2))
 (segment (start 122.9351 104.5256) (end 122.9351 105.5996) (width 0.254) (layer "F.Cu") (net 2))
 (segment (start 125.1632 106.7206) (end 124.558 106.1154) (width 0.254) (layer "F.Cu") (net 2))
 (segment (start 128.3741 107.3556) (end 128.9431 107.9246) (width 0.254) (layer "F.Cu") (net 2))
 (segment (start 125.6411 98.7258) (end 125.5689 98.7258) (width 0.254) (layer "F.Cu") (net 2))
 (segment (start 122.2121 99.7966) (end 122.9851 99.7966) (width 0.254) (layer "F.Cu") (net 2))
 (segment (start 121.2351 101.9166) (end 122.2121 100.9396) (width 0.254) (layer "F.Cu") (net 2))
 (segment (start 129.2385 104.906) (end 129.1771 104.8446) (width 0.254) (layer "F.Cu") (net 2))
 (via (at 130.0861 104.906) (size 0.9064) (drill 0.5) (layers "F.Cu" "B.Cu") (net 2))
 (via (at 125.6411 98.7258) (size 0.9064) (drill 0.5) (layers "F.Cu" "B.Cu") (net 2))
 (via (at 129.0701 107.9246) (size 0.9064) (drill 0.5) (layers "F.Cu" "B.Cu") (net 2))
 (segment (start 129.0701 105.6386) (end 129.0701 107.9246) (width 0.254) (layer "B.Cu") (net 2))
 (segment (start 127.1103 98.7258) (end 128.9431 100.5586) (width 0.254) (layer "B.Cu") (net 2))
 (segment (start 128.9431 103.8606) (end 130.0861 105.0036) (width 0.254) (layer "B.Cu") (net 2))
 (segment (start 128.9431 100.5586) (end 128.9431 103.8606) (width 0.254) (layer "B.Cu") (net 2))
 (segment (start 129.7051 105.0036) (end 130.0861 105.0036) (width 0.254) (layer "B.Cu") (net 2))
 (segment (start 129.7051 105.0036) (end 129.0701 105.6386) (width 0.254) (layer "B.Cu") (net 2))
 (segment (start 130.0861 104.906) (end 130.0861 105.0036) (width 0.254) (layer "B.Cu") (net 2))
 (segment (start 127.1103 98.7258) (end 125.6411 98.7258) (width 0.254) (layer "B.Cu") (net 2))
 (segment (start 125.9271 104.0946) (end 125.9271 104.9716) (width 0.254) (layer "F.Cu") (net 25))
 (segment (start 125.9271 104.9716) (end 125.5141 105.3846) (width 0.254) (layer "F.Cu") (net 25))
 (via (at 125.5141 105.3846) (size 0.9064) (drill 0.5) (layers "F.Cu" "B.Cu") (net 25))
 (segment (start 125.5141 105.3846) (end 125.5141 106.1466) (width 0.254) (layer "B.Cu") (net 25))
 (segment (start 126.2761 106.9086) (end 125.5141 106.1466) (width 0.254) (layer "B.Cu") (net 25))
 (segment (start 124.7861 110.2106) (end 125.3155 109.6812) (width 0.254) (layer "F.Cu") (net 11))
 (segment (start 125.927412 109.6812) (end 125.3155 109.6812) (width 0.254) (layer "F.Cu") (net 11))
 (segment (start 125.9271 103.5946) (end 125.0181 103.5946) (width 0.254) (layer "F.Cu") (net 11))
 (segment (start 125.0181 103.5946) (end 124.4981 104.1146) (width 0.254) (layer "F.Cu") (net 11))
 (segment (start 126.054412 109.5542) (end 125.927412 109.6812) (width 0.254) (layer "F.Cu") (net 11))
 (via (at 124.4981 104.1146) (size 0.9064) (drill 0.5) (layers "F.Cu" "B.Cu") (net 11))
 (via (at 126.054412 109.5542) (size 0.9064) (drill 0.5) (layers "F.Cu" "B.Cu") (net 11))
 (segment (start 124.4981 104.1146) (end 124.4981 107.997888) (width 0.254) (layer "B.Cu") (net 11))
 (segment (start 126.054412 109.5542) (end 124.4981 107.997888) (width 0.254) (layer "B.Cu") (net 11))
 (segment (start 122.6861 110.2106) (end 121.1571 110.2106) (width 0.254) (layer "F.Cu") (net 10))
 (segment (start 120.0341 103.6256) (end 121.2351 103.6256) (width 0.254) (layer "F.Cu") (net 3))
 (segment (start 119.6561 104.0036) (end 120.0341 103.6256) (width 0.254) (layer "F.Cu") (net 3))
 (segment (start 113.8087 102.585919) (end 113.826418 102.603638) (width 0.254) (layer "F.Cu") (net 3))
 (segment (start 122.9851 99.0466) (end 123.7963 99.0466) (width 0.254) (layer "F.Cu") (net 3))
 (segment (start 113.826418 103.474919) (end 114.3551 104.0036) (width 0.254) (layer "F.Cu") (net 3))
 (segment (start 124.1171 98.7258) (end 123.7963 99.0466) (width 0.254) (layer "F.Cu") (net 3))
 (segment (start 117.6571 104.0036) (end 119.6561 104.0036) (width 0.254) (layer "F.Cu") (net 3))
 (segment (start 114.3551 104.0036) (end 117.6571 104.0036) (width 0.254) (layer "F.Cu") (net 3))
 (segment (start 113.826418 102.603638) (end 113.826418 103.474919) (width 0.254) (layer "F.Cu") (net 3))
 (via (at 113.8087 102.585919) (size 0.9064) (drill 0.5) (layers "F.Cu" "B.Cu") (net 3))
 (via (at 124.1171 98.7258) (size 0.9064) (drill 0.5) (layers "F.Cu" "B.Cu") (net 3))
 (segment (start 124.1171 98.7258) (end 117.6949 98.7258) (width 0.254) (layer "B.Cu") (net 3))
 (segment (start 117.6949 98.7258) (end 113.834781 102.585919) (width 0.254) (layer "B.Cu") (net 3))
 (segment (start 113.834781 102.585919) (end 113.8087 102.585919) (width 0.254) (layer "B.Cu") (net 3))
 (segment (start 120.1801 102.8446) (end 119.5451 102.2096) (width 0.254) (layer "F.Cu") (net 5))
 (segment (start 119.5451 102.0036) (end 117.6571 102.0036) (width 0.254) (layer "F.Cu") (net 5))
 (segment (start 119.5451 102.1306) (end 119.5451 102.0036) (width 0.254) (layer "F.Cu") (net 5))
 (segment (start 121.2161 102.8446) (end 120.1801 102.8446) (width 0.254) (layer "F.Cu") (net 5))
 (segment (start 119.6011 102.1306) (end 119.5451 102.1306) (width 0.254) (layer "F.Cu") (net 5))
 (segment (start 119.5451 102.2096) (end 119.5451 102.1306) (width 0.254) (layer "F.Cu") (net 5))
 (segment (start 121.1851 100.5466) (end 119.6011 102.1306) (width 0.254) (layer "F.Cu") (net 5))
 (segment (start 121.2161 102.8446) (end 121.2351 102.8256) (width 0.254) (layer "F.Cu") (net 5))
 (segment (start 124.4941 103.0946) (end 123.3251 101.9256) (width 0.254) (layer "F.Cu") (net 1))
 (segment (start 123.3251 101.9256) (end 122.9351 101.9256) (width 0.254) (layer "F.Cu") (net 1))
 (segment (start 122.9851 100.5466) (end 122.9351 100.5966) (width 0.254) (layer "F.Cu") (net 1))
 (segment (start 125.9271 103.0946) (end 124.4941 103.0946) (width 0.254) (layer "F.Cu") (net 1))
 (segment (start 122.9351 100.5966) (end 122.9351 101.9256) (width 0.254) (layer "F.Cu") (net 1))
 (segment (start 119.7831 106.0036) (end 120.6271 106.8476) (width 0.254) (layer "F.Cu") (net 9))
 (segment (start 123.071 108.6206) (end 124.3101 108.6206) (width 0.254) (layer "F.Cu") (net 9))
 (segment (start 121.3231 106.8476) (end 121.3891 106.7816) (width 0.254) (layer "F.Cu") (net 9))
 (segment (start 122.9351 103.2256) (end 122.0851 103.2256) (width 0.254) (layer "F.Cu") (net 9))
 (segment (start 123.2281 106.7816) (end 123.0351 106.7816) (width 0.254) (layer "F.Cu") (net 9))
 (segment (start 121.3891 106.7816) (end 123.0351 106.7816) (width 0.254) (layer "F.Cu") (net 9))
 (segment (start 122.0851 105.7347) (end 123.071 106.7206) (width 0.254) (layer "F.Cu") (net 9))
 (segment (start 122.9351 103.2256) (end 122.9351 103.6256) (width 0.254) (layer "F.Cu") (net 9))
 (segment (start 122.0851 103.2256) (end 122.0851 105.7347) (width 0.254) (layer "F.Cu") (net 9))
 (segment (start 124.3711 108.5596) (end 124.3711 106.7816) (width 0.254) (layer "F.Cu") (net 9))
 (segment (start 124.3101 108.6206) (end 124.3711 108.5596) (width 0.254) (layer "F.Cu") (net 9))
 (segment (start 123.0351 106.7816) (end 122.9741 106.7206) (width 0.254) (layer "F.Cu") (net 9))
 (segment (start 122.9351 102.8256) (end 122.9351 103.2256) (width 0.254) (layer "F.Cu") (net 9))
 (segment (start 124.3711 106.7816) (end 123.2281 106.7816) (width 0.254) (layer "F.Cu") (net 9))
 (segment (start 120.6271 106.8476) (end 121.3231 106.8476) (width 0.254) (layer "F.Cu") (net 9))
 (segment (start 117.6571 106.0036) (end 119.7831 106.0036) (width 0.254) (layer "F.Cu") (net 9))
 (segment (start 122.9741 106.7206) (end 123.071 106.7206) (width 0.254) (layer "F.Cu") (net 9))
 (segment (start 121.1851 99.0466) (end 120.6761 99.0466) (width 0.254) (layer "F.Cu") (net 4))
 (segment (start 125.1063 102.5946) (end 124.3497 101.838) (width 0.254) (layer "F.Cu") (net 4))
 (segment (start 121.2351 104.5256) (end 120.766387 104.994313) (width 0.254) (layer "F.Cu") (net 4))
 (segment (start 120.6761 99.0466) (end 118.9101 100.8126) (width 0.254) (layer "F.Cu") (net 4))
 (segment (start 120.766387 104.994313) (end 120.766387 105.5116) (width 0.254) (layer "F.Cu") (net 4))
 (segment (start 125.9271 102.5946) (end 125.1063 102.5946) (width 0.254) (layer "F.Cu") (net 4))
 (via (at 120.766387 105.5116) (size 0.9064) (drill 0.5) (layers "F.Cu" "B.Cu") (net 4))
 (via (at 118.9101 100.8126) (size 0.9064) (drill 0.5) (layers "F.Cu" "B.Cu") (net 4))
 (via (at 124.3497 101.838) (size 0.9064) (drill 0.5) (layers "F.Cu" "B.Cu") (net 4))
 (segment (start 121.8217 101.838) (end 120.766387 102.893313) (width 0.254) (layer "B.Cu") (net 4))
 (segment (start 120.766387 102.893313) (end 120.766387 105.5116) (width 0.254) (layer "B.Cu") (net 4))
 (segment (start 118.9101 100.8126) (end 118.9101 103.655313) (width 0.254) (layer "B.Cu") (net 4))
 (segment (start 124.3497 101.838) (end 121.8217 101.838) (width 0.254) (layer "B.Cu") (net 4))
 (segment (start 118.9101 103.655313) (end 120.766387 105.5116) (width 0.254) (layer "B.Cu") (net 4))
 (segment (start 125.2601 100.4196) (end 125.2601 100.199) (width 0.254) (layer "F.Cu") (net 23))
 (segment (start 125.9271 101.0866) (end 125.2601 100.4196) (width 0.254) (layer "F.Cu") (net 23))
 (segment (start 125.9271 101.5946) (end 125.9271 101.0866) (width 0.254) (layer "F.Cu") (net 23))
 (via (at 125.2601 100.199) (size 0.9064) (drill 0.5) (layers "F.Cu" "B.Cu") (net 23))
 (segment (start 123.2495 99.437) (end 123.6091 99.7966) (width 0.254) (layer "B.Cu") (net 23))
 (segment (start 124.8577 99.7966) (end 125.2601 100.199) (width 0.254) (layer "B.Cu") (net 23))
 (segment (start 117.0051 100.062182) (end 117.630281 99.437) (width 0.254) (layer "B.Cu") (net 23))
 (segment (start 123.6091 99.7966) (end 124.8577 99.7966) (width 0.254) (layer "B.Cu") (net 23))
 (segment (start 117.0051 103.8606) (end 117.0051 100.062182) (width 0.254) (layer "B.Cu") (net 23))
 (segment (start 117.630281 99.437) (end 123.2495 99.437) (width 0.254) (layer "B.Cu") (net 23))
 (segment (start 124.6679 100.7284) (end 124.267912 100.7284) (width 0.254) (layer "F.Cu") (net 24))
 (segment (start 125.461131 102.0946) (end 125.1331 101.766569) (width 0.254) (layer "F.Cu") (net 24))
 (segment (start 125.1331 101.1936) (end 124.6679 100.7284) (width 0.254) (layer "F.Cu") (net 24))
 (segment (start 125.9271 102.0946) (end 125.461131 102.0946) (width 0.254) (layer "F.Cu") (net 24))
 (segment (start 125.1331 101.766569) (end 125.1331 101.1936) (width 0.254) (layer "F.Cu") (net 24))
 (via (at 124.267912 100.7284) (size 0.9064) (drill 0.5) (layers "F.Cu" "B.Cu") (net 24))
 (segment (start 117.0051 106.4006) (end 117.7671 105.6386) (width 0.254) (layer "B.Cu") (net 24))
 (segment (start 124.236693 100.697182) (end 124.267912 100.7284) (width 0.254) (layer "B.Cu") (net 24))
 (segment (start 117.7671 105.6386) (end 117.7671 100.1776) (width 0.254) (layer "B.Cu") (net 24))
 (segment (start 117.7671 100.1776) (end 118.0505 99.8942) (width 0.254) (layer "B.Cu") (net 24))
 (segment (start 122.784718 99.8942) (end 123.5877 100.697182) (width 0.254) (layer "B.Cu") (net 24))
 (segment (start 123.5877 100.697182) (end 124.236693 100.697182) (width 0.254) (layer "B.Cu") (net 24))
 (segment (start 118.0505 99.8942) (end 122.784718 99.8942) (width 0.254) (layer "B.Cu") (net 24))
 (segment (start 129.9271 103.0946) (end 131.6061 103.0946) (width 0.254) (layer "F.Cu") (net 6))
 (segment (start 131.6061 103.0946) (end 133.8961 105.3846) (width 0.254) (layer "F.Cu") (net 6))
 (segment (start 136.0551 105.3846) (end 133.8961 105.3846) (width 0.254) (layer "F.Cu") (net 6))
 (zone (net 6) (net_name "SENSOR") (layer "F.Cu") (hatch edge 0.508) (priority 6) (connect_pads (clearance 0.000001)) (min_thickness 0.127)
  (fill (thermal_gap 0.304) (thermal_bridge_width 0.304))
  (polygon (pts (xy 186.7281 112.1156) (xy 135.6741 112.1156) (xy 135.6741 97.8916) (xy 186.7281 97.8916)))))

